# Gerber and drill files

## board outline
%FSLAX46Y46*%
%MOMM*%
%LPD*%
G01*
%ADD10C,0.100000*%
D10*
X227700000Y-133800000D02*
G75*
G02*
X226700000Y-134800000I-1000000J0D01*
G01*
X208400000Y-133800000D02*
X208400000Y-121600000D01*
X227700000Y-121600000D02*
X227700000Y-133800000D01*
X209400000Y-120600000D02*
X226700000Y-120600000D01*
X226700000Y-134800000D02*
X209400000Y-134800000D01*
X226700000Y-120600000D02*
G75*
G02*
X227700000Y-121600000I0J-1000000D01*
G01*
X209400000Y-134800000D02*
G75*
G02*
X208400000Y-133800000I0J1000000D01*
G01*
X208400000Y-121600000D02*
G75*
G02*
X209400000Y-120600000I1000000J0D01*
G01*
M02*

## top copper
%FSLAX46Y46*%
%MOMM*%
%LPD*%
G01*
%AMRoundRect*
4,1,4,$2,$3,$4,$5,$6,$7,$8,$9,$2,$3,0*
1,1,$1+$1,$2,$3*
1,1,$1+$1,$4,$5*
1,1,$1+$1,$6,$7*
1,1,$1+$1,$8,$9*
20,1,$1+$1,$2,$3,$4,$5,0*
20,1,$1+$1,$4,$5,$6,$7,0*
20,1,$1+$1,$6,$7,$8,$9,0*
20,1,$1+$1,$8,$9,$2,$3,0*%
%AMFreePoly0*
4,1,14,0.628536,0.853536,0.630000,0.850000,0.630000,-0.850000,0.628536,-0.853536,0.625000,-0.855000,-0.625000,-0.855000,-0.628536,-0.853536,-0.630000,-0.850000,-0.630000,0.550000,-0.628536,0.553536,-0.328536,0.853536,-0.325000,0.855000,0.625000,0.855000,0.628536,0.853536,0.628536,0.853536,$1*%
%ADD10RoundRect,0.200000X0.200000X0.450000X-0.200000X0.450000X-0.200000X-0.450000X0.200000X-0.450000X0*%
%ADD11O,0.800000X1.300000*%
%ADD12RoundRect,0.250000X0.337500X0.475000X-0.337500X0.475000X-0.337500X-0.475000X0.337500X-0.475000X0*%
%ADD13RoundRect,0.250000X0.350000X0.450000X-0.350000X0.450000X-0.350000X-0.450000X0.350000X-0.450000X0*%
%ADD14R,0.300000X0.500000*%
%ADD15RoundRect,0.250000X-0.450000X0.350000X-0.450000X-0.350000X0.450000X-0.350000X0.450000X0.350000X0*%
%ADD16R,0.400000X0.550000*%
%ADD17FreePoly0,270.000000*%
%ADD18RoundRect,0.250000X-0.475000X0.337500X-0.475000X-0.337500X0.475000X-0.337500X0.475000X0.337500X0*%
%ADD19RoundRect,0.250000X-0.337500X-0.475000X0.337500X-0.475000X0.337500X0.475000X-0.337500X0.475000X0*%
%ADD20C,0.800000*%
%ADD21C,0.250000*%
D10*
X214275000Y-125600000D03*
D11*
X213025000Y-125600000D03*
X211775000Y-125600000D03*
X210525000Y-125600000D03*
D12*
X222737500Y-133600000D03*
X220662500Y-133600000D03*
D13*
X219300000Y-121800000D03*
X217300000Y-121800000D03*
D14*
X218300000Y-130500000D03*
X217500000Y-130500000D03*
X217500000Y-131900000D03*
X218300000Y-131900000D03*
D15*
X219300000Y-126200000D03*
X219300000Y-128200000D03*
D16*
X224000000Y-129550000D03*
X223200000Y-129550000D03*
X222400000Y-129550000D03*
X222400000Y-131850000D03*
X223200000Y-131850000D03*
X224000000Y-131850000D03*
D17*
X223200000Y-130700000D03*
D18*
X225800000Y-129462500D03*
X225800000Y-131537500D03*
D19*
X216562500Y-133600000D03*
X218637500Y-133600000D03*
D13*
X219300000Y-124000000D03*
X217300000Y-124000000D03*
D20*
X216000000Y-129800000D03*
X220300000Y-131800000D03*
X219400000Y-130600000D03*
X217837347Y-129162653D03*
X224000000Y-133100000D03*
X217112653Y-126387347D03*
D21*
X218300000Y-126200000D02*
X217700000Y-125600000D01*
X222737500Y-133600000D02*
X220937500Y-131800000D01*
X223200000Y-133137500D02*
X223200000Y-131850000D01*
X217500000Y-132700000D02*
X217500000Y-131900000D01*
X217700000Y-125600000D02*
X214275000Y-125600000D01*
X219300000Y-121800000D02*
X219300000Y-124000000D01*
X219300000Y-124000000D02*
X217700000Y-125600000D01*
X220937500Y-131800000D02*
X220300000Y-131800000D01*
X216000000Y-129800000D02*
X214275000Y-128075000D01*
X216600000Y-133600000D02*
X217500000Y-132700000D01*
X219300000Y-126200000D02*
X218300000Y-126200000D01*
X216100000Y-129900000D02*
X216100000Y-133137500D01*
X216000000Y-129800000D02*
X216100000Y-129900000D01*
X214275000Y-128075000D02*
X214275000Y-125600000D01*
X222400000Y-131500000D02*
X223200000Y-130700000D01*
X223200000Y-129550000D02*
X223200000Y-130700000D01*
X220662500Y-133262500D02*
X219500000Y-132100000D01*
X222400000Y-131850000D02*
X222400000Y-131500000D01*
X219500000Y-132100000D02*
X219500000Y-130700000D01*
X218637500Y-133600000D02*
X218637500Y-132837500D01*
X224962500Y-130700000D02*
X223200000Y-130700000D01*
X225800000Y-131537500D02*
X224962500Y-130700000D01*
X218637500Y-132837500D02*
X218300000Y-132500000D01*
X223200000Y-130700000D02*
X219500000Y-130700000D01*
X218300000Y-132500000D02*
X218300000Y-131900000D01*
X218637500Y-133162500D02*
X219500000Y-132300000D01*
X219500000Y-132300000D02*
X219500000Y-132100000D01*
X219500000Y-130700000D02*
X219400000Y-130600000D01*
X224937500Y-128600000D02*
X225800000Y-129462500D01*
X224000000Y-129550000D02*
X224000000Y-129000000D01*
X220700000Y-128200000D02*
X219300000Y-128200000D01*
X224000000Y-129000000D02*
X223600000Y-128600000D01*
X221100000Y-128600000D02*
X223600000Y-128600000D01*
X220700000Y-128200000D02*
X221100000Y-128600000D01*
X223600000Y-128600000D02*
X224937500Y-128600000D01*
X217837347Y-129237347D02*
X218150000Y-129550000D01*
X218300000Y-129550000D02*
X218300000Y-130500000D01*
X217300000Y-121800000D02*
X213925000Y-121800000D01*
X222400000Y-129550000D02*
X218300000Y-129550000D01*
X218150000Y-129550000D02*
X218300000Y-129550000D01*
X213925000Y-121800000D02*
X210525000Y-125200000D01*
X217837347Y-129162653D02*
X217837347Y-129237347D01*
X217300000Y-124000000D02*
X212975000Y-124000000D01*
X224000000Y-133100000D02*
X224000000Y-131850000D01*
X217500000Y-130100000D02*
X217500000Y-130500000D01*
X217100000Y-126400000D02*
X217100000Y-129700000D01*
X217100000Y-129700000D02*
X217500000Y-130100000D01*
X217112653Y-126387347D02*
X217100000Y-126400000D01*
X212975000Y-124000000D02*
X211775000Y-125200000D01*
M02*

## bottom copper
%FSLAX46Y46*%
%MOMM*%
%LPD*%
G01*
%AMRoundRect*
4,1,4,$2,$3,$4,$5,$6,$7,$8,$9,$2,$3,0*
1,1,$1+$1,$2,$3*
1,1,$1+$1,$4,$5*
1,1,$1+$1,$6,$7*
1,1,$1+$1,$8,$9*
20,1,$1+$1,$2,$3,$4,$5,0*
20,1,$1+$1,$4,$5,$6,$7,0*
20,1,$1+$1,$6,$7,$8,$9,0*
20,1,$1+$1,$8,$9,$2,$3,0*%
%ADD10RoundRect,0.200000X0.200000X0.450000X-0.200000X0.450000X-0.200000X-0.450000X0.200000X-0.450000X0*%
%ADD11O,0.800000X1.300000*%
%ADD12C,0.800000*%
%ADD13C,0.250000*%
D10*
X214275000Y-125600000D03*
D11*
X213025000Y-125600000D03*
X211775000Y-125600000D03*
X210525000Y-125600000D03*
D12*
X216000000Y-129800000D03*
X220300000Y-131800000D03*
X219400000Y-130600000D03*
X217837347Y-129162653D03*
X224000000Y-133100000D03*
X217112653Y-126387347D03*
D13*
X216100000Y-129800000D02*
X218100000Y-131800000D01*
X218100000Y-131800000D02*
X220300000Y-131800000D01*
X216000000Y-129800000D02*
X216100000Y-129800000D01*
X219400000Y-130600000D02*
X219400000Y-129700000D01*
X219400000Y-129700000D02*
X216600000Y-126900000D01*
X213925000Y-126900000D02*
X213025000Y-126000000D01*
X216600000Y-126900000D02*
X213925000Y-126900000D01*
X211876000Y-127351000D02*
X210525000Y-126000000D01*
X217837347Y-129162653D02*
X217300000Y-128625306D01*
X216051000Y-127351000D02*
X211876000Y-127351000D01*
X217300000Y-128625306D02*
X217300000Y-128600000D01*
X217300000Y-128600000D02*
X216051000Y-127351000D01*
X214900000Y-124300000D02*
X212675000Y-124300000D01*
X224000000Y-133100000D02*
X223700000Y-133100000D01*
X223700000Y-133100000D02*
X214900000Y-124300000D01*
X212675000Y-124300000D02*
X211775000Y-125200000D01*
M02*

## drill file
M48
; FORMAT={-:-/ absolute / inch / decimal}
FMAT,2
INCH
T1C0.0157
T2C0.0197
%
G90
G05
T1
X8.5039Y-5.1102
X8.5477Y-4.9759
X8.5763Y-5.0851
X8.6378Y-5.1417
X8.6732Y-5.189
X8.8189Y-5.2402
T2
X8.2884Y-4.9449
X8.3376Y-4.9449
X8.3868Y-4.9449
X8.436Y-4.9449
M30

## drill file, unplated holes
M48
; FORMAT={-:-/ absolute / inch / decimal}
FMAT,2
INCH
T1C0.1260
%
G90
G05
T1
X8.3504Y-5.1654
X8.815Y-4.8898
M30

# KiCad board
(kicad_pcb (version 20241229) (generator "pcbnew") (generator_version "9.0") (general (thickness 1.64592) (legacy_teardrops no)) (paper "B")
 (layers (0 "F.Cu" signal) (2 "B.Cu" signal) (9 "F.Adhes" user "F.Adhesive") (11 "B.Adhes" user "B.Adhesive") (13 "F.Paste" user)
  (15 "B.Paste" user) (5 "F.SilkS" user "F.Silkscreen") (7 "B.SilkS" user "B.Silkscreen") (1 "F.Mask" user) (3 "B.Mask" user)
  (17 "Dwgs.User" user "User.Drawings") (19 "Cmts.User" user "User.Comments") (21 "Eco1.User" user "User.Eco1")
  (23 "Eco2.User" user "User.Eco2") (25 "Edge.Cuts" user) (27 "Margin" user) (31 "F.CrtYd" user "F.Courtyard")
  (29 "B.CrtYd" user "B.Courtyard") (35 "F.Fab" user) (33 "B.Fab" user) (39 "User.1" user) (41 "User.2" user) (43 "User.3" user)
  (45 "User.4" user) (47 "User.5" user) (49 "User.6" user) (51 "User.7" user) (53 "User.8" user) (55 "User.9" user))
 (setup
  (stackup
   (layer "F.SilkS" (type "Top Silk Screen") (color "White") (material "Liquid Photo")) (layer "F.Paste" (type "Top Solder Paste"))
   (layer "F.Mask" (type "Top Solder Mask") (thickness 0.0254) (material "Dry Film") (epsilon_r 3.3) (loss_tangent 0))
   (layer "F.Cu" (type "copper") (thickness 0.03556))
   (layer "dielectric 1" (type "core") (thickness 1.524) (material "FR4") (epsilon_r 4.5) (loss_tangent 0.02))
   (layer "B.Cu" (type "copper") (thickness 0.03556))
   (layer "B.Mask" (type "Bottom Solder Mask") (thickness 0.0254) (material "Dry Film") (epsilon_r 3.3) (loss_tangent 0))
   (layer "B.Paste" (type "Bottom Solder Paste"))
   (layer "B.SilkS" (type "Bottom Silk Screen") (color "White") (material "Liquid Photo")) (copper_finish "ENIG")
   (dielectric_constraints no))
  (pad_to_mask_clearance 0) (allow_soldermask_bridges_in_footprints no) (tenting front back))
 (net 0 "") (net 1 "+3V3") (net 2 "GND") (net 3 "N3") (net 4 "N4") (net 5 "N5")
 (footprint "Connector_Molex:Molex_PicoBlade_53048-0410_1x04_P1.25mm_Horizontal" (layer "F.Cu") (at 214.275 125.6 180)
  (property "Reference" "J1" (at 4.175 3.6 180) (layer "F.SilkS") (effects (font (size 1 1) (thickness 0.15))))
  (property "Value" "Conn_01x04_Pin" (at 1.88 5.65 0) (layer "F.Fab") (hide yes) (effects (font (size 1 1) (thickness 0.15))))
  (pad "1" thru_hole roundrect (at 0 0 180) (size 0.8 1.3) (drill 0.5) (layers "*.Cu" "*.Mask") (remove_unused_layers no)
   (roundrect_rratio 0.25) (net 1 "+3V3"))
  (pad "2" thru_hole oval (at 1.25 0 180) (size 0.8 1.3) (drill 0.5) (layers "*.Cu" "*.Mask") (remove_unused_layers no) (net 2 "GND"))
  (pad "3" thru_hole oval (at 2.5 0 180) (size 0.8 1.3) (drill 0.5) (layers "*.Cu" "*.Mask") (remove_unused_layers no) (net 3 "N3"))
  (pad "4" thru_hole oval (at 3.75 0 180) (size 0.8 1.3) (drill 0.5) (layers "*.Cu" "*.Mask") (remove_unused_layers no) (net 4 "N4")))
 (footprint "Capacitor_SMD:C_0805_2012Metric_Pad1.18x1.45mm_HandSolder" (layer "F.Cu") (at 221.7 133.6 180)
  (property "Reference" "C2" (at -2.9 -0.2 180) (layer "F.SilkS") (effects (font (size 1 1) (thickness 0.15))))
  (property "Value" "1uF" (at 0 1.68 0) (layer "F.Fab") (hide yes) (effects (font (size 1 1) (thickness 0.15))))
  (pad "1" smd roundrect (at -1.0375 0 180) (size 1.175 1.45) (layers "F.Cu" "F.Mask" "F.Paste") (roundrect_rratio 0.212766) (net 1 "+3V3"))
  (pad "2" smd roundrect (at 1.0375 0 180) (size 1.175 1.45) (layers "F.Cu" "F.Mask" "F.Paste") (roundrect_rratio 0.212766) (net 2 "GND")))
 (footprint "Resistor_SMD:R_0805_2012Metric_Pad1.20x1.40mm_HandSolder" (layer "F.Cu") (at 218.3 121.8 180)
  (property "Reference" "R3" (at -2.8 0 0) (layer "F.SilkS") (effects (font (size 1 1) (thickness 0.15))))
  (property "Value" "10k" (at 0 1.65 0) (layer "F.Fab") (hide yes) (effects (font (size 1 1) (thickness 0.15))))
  (pad "1" smd roundrect (at -1 0 180) (size 1.2 1.4) (layers "F.Cu" "F.Mask" "F.Paste") (roundrect_rratio 0.208333) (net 1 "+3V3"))
  (pad "2" smd roundrect (at 1 0 180) (size 1.2 1.4) (layers "F.Cu" "F.Mask" "F.Paste") (roundrect_rratio 0.208333) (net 4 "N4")))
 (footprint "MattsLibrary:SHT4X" (layer "F.Cu") (at 217.9 131.2 -90)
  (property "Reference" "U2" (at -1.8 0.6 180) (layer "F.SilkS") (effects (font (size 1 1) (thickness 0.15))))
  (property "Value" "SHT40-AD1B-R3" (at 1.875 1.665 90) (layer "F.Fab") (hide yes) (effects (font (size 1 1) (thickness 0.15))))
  (pad "1" smd rect (at -0.7 -0.4 270) (size 0.5 0.3) (layers "F.Cu" "F.Mask" "F.Paste") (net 4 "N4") (solder_mask_margin 0.102))
  (pad "2" smd rect (at -0.7 0.4 270) (size 0.5 0.3) (layers "F.Cu" "F.Mask" "F.Paste") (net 3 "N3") (solder_mask_margin 0.102))
  (pad "3" smd rect (at 0.7 0.4 270) (size 0.5 0.3) (layers "F.Cu" "F.Mask" "F.Paste") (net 1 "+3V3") (solder_mask_margin 0.102))
  (pad "4" smd rect (at 0.7 -0.4 270) (size 0.5 0.3) (layers "F.Cu" "F.Mask" "F.Paste") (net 2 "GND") (solder_mask_margin 0.102)))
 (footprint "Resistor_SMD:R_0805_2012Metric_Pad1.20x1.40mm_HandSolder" (layer "F.Cu") (at 219.3 127.2 -90)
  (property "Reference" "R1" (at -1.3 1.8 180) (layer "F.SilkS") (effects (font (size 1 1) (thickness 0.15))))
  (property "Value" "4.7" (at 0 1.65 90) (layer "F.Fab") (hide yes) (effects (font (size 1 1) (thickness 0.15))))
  (pad "1" smd roundrect (at -1 0 270) (size 1.2 1.4) (layers "F.Cu" "F.Mask" "F.Paste") (roundrect_rratio 0.208333) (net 1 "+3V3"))
  (pad "2" smd roundrect (at 1 0 270) (size 1.2 1.4) (layers "F.Cu" "F.Mask" "F.Paste") (roundrect_rratio 0.208333) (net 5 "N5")))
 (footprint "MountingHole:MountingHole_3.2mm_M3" (layer "F.Cu") (at 223.9 124.2)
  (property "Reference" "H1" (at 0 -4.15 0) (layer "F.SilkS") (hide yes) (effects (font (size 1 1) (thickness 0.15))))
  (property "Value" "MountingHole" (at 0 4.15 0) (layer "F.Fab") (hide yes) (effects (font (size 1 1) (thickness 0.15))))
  (pad "" np_thru_hole circle (at 0 0) (size 3.2 3.2) (drill 3.2) (layers "*.Cu" "*.Mask")))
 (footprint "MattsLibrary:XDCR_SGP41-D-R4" (layer "F.Cu") (at 223.2 130.7 -90)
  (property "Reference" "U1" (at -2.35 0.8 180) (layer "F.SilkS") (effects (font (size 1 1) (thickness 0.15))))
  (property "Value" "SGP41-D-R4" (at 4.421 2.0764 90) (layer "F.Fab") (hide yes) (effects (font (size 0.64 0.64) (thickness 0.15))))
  (pad "1" smd rect (at -1.15 -0.8 270) (size 0.55 0.4) (layers "F.Cu" "F.Mask" "F.Paste") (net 5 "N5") (solder_mask_margin 0.102))
  (pad "2" smd rect (at -1.15 0 270) (size 0.55 0.4) (layers "F.Cu" "F.Mask" "F.Paste") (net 2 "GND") (solder_mask_margin 0.102))
  (pad "3" smd rect (at -1.15 0.8 270) (size 0.55 0.4) (layers "F.Cu" "F.Mask" "F.Paste") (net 4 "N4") (solder_mask_margin 0.102))
  (pad "4" smd rect (at 1.15 0.8 270) (size 0.55 0.4) (layers "F.Cu" "F.Mask" "F.Paste") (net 2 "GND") (solder_mask_margin 0.102))
  (pad "5" smd rect (at 1.15 0 270) (size 0.55 0.4) (layers "F.Cu" "F.Mask" "F.Paste") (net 1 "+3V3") (solder_mask_margin 0.102))
  (pad "6" smd rect (at 1.15 -0.8 270) (size 0.55 0.4) (layers "F.Cu" "F.Mask" "F.Paste") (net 3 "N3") (solder_mask_margin 0.102))
  (pad "7" smd custom (at 0 0 270) (size 0.5 0.5) (layers "F.Cu") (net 2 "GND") (options (clearance outline) (anchor rect)) (primitives)))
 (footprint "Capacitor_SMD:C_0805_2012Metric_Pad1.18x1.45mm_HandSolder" (layer "F.Cu") (at 225.8 130.5 -90)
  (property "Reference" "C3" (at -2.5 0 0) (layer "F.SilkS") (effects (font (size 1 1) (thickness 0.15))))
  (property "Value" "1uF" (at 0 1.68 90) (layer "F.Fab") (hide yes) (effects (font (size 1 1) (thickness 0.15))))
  (pad "1" smd roundrect (at -1.0375 0 270) (size 1.175 1.45) (layers "F.Cu" "F.Mask" "F.Paste") (roundrect_rratio 0.212766) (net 5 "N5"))
  (pad "2" smd roundrect (at 1.0375 0 270) (size 1.175 1.45) (layers "F.Cu" "F.Mask" "F.Paste") (roundrect_rratio 0.212766) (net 2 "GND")))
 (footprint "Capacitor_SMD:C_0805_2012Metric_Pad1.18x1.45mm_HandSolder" (layer "F.Cu") (at 217.6 133.6)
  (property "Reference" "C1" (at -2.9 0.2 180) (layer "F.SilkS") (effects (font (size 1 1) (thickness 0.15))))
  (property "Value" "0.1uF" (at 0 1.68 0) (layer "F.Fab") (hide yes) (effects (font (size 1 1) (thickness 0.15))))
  (pad "1" smd roundrect (at -1.0375 0) (size 1.175 1.45) (layers "F.Cu" "F.Mask" "F.Paste") (roundrect_rratio 0.212766) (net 1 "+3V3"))
  (pad "2" smd roundrect (at 1.0375 0) (size 1.175 1.45) (layers "F.Cu" "F.Mask" "F.Paste") (roundrect_rratio 0.212766) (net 2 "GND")))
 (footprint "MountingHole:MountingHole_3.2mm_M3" (layer "F.Cu") (at 212.1 131.2)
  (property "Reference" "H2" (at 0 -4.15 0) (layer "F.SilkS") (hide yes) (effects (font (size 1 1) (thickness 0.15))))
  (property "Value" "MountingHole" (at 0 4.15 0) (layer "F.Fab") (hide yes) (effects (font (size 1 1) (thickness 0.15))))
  (pad "" np_thru_hole circle (at 0 0) (size 3.2 3.2) (drill 3.2) (layers "*.Cu" "*.Mask")))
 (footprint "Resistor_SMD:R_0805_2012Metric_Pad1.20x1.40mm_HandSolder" (layer "F.Cu") (at 218.3 124 180)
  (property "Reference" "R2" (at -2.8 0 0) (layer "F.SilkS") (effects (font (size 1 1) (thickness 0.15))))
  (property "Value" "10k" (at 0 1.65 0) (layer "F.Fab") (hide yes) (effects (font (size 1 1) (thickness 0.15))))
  (pad "1" smd roundrect (at -1 0 180) (size 1.2 1.4) (layers "F.Cu" "F.Mask" "F.Paste") (roundrect_rratio 0.208333) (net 1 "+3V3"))
  (pad "2" smd roundrect (at 1 0 180) (size 1.2 1.4) (layers "F.Cu" "F.Mask" "F.Paste") (roundrect_rratio 0.208333) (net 3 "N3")))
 (gr_arc (start 227.7 133.8) (mid 227.407107 134.507107) (end 226.7 134.8) (stroke (width 0.1) (type default)) (layer "Edge.Cuts"))
 (gr_line (start 208.4 133.8) (end 208.4 121.6) (stroke (width 0.1) (type default)) (layer "Edge.Cuts"))
 (gr_line (start 227.7 121.6) (end 227.7 133.8) (stroke (width 0.1) (type default)) (layer "Edge.Cuts"))
 (gr_line (start 209.4 120.6) (end 226.7 120.6) (stroke (width 0.1) (type default)) (layer "Edge.Cuts"))
 (gr_line (start 226.7 134.8) (end 209.4 134.8) (stroke (width 0.1) (type default)) (layer "Edge.Cuts"))
 (gr_arc (start 226.7 120.6) (mid 227.407107 120.892893) (end 227.7 121.6) (stroke (width 0.1) (type default)) (layer "Edge.Cuts"))
 (gr_arc (start 209.4 134.8) (mid 208.692893 134.507107) (end 208.4 133.8) (stroke (width 0.1) (type default)) (layer "Edge.Cuts"))
 (gr_arc (start 208.4 121.6) (mid 208.692893 120.892893) (end 209.4 120.6) (stroke (width 0.1) (type default)) (layer "Edge.Cuts"))
 (segment (start 218.3 126.2) (end 217.7 125.6) (width 0.25) (layer "F.Cu") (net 1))
 (segment (start 222.7375 133.6) (end 220.9375 131.8) (width 0.25) (layer "F.Cu") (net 1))
 (segment (start 223.2 133.1375) (end 223.2 131.85) (width 0.25) (layer "F.Cu") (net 1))
 (segment (start 217.5 132.7) (end 217.5 131.9) (width 0.25) (layer "F.Cu") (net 1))
 (segment (start 217.7 125.6) (end 214.275 125.6) (width 0.25) (layer "F.Cu") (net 1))
 (segment (start 219.3 121.8) (end 219.3 124) (width 0.25) (layer "F.Cu") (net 1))
 (segment (start 219.3 124) (end 217.7 125.6) (width 0.25) (layer "F.Cu") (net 1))
 (segment (start 220.9375 131.8) (end 220.3 131.8) (width 0.25) (layer "F.Cu") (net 1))
 (segment (start 216 129.8) (end 214.275 128.075) (width 0.25) (layer "F.Cu") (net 1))
 (segment (start 216.6 133.6) (end 217.5 132.7) (width 0.25) (layer "F.Cu") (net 1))
 (segment (start 219.3 126.2) (end 218.3 126.2) (width 0.25) (layer "F.Cu") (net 1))
 (segment (start 216.1 129.9) (end 216.1 133.1375) (width 0.25) (layer "F.Cu") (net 1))
 (segment (start 216 129.8) (end 216.1 129.9) (width 0.25) (layer "F.Cu") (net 1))
 (segment (start 214.275 128.075) (end 214.275 125.6) (width 0.25) (layer "F.Cu") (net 1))
 (via (at 216 129.8) (size 0.8) (drill 0.4) (layers "F.Cu" "B.Cu") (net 1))
 (via (at 220.3 131.8) (size 0.8) (drill 0.4) (layers "F.Cu" "B.Cu") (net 1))
 (segment (start 216.1 129.8) (end 218.1 131.8) (width 0.25) (layer "B.Cu") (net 1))
 (segment (start 218.1 131.8) (end 220.3 131.8) (width 0.25) (layer "B.Cu") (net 1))
 (segment (start 216 129.8) (end 216.1 129.8) (width 0.25) (layer "B.Cu") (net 1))
 (segment (start 222.4 131.5) (end 223.2 130.7) (width 0.25) (layer "F.Cu") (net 2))
 (segment (start 223.2 129.55) (end 223.2 130.7) (width 0.25) (layer "F.Cu") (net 2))
 (segment (start 220.6625 133.2625) (end 219.5 132.1) (width 0.25) (layer "F.Cu") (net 2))
 (segment (start 222.4 131.85) (end 222.4 131.5) (width 0.25) (layer "F.Cu") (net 2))
 (segment (start 219.5 132.1) (end 219.5 130.7) (width 0.25) (layer "F.Cu") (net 2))
 (segment (start 218.6375 133.6) (end 218.6375 132.8375) (width 0.25) (layer "F.Cu") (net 2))
 (segment (start 224.9625 130.7) (end 223.2 130.7) (width 0.25) (layer "F.Cu") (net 2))
 (segment (start 225.8 131.5375) (end 224.9625 130.7) (width 0.25) (layer "F.Cu") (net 2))
 (segment (start 218.6375 132.8375) (end 218.3 132.5) (width 0.25) (layer "F.Cu") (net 2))
 (segment (start 223.2 130.7) (end 219.5 130.7) (width 0.25) (layer "F.Cu") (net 2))
 (segment (start 218.3 132.5) (end 218.3 131.9) (width 0.25) (layer "F.Cu") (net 2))
 (segment (start 218.6375 133.1625) (end 219.5 132.3) (width 0.25) (layer "F.Cu") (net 2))
 (segment (start 219.5 132.3) (end 219.5 132.1) (width 0.25) (layer "F.Cu") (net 2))
 (segment (start 219.5 130.7) (end 219.4 130.6) (width 0.25) (layer "F.Cu") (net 2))
 (via (at 219.4 130.6) (size 0.8) (drill 0.4) (layers "F.Cu" "B.Cu") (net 2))
 (segment (start 219.4 130.6) (end 219.4 129.7) (width 0.25) (layer "B.Cu") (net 2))
 (segment (start 219.4 129.7) (end 216.6 126.9) (width 0.25) (layer "B.Cu") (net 2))
 (segment (start 213.925 126.9) (end 213.025 126) (width 0.25) (layer "B.Cu") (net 2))
 (segment (start 216.6 126.9) (end 213.925 126.9) (width 0.25) (layer "B.Cu") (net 2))
 (segment (start 224.9375 128.6) (end 225.8 129.4625) (width 0.25) (layer "F.Cu") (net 5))
 (segment (start 224 129.55) (end 224 129) (width 0.25) (layer "F.Cu") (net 5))
 (segment (start 220.7 128.2) (end 219.3 128.2) (width 0.25) (layer "F.Cu") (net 5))
 (segment (start 224 129) (end 223.6 128.6) (width 0.25) (layer "F.Cu") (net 5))
 (segment (start 221.1 128.6) (end 223.6 128.6) (width 0.25) (layer "F.Cu") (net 5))
 (segment (start 220.7 128.2) (end 221.1 128.6) (width 0.25) (layer "F.Cu") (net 5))
 (segment (start 223.6 128.6) (end 224.9375 128.6) (width 0.25) (layer "F.Cu") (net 5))
 (segment (start 217.837347 129.237347) (end 218.15 129.55) (width 0.25) (layer "F.Cu") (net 4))
 (segment (start 218.3 129.55) (end 218.3 130.5) (width 0.25) (layer "F.Cu") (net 4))
 (segment (start 217.3 121.8) (end 213.925 121.8) (width 0.25) (layer "F.Cu") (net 4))
 (segment (start 222.4 129.55) (end 218.3 129.55) (width 0.25) (layer "F.Cu") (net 4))
 (segment (start 218.15 129.55) (end 218.3 129.55) (width 0.25) (layer "F.Cu") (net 4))
 (segment (start 213.925 121.8) (end 210.525 125.2) (width 0.25) (layer "F.Cu") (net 4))
 (segment (start 217.837347 129.162653) (end 217.837347 129.237347) (width 0.25) (layer "F.Cu") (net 4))
 (via (at 217.837347 129.162653) (size 0.8) (drill 0.4) (layers "F.Cu" "B.Cu") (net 4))
 (segment (start 211.876 127.351) (end 210.525 126) (width 0.25) (layer "B.Cu") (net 4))
 (segment (start 217.837347 129.162653) (end 217.3 128.625306) (width 0.25) (layer "B.Cu") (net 4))
 (segment (start 216.051 127.351) (end 211.876 127.351) (width 0.25) (layer "B.Cu") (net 4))
 (segment (start 217.3 128.625306) (end 217.3 128.6) (width 0.25) (layer "B.Cu") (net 4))
 (segment (start 217.3 128.6) (end 216.051 127.351) (width 0.25) (layer "B.Cu") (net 4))
 (segment (start 217.3 124) (end 212.975 124) (width 0.25) (layer "F.Cu") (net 3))
 (segment (start 224 133.1) (end 224 131.85) (width 0.25) (layer "F.Cu") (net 3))
 (segment (start 217.5 130.1) (end 217.5 130.5) (width 0.25) (layer "F.Cu") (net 3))
 (segment (start 217.1 126.4) (end 217.1 129.7) (width 0.25) (layer "F.Cu") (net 3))
 (segment (start 217.1 129.7) (end 217.5 130.1) (width 0.25) (layer "F.Cu") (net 3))
 (segment (start 217.112653 126.387347) (end 217.1 126.4) (width 0.25) (layer "F.Cu") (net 3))
 (segment (start 212.975 124) (end 211.775 125.2) (width 0.25) (layer "F.Cu") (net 3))
 (via (at 224 133.1) (size 0.8) (drill 0.4) (layers "F.Cu" "B.Cu") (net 3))
 (via (at 217.112653 126.387347) (size 0.8) (drill 0.4) (layers "F.Cu" "B.Cu") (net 3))
 (segment (start 214.9 124.3) (end 212.675 124.3) (width 0.25) (layer "B.Cu") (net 3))
 (segment (start 224 133.1) (end 223.7 133.1) (width 0.25) (layer "B.Cu") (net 3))
 (segment (start 223.7 133.1) (end 214.9 124.3) (width 0.25) (layer "B.Cu") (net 3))
 (segment (start 212.675 124.3) (end 211.775 125.2) (width 0.25) (layer "B.Cu") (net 3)))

